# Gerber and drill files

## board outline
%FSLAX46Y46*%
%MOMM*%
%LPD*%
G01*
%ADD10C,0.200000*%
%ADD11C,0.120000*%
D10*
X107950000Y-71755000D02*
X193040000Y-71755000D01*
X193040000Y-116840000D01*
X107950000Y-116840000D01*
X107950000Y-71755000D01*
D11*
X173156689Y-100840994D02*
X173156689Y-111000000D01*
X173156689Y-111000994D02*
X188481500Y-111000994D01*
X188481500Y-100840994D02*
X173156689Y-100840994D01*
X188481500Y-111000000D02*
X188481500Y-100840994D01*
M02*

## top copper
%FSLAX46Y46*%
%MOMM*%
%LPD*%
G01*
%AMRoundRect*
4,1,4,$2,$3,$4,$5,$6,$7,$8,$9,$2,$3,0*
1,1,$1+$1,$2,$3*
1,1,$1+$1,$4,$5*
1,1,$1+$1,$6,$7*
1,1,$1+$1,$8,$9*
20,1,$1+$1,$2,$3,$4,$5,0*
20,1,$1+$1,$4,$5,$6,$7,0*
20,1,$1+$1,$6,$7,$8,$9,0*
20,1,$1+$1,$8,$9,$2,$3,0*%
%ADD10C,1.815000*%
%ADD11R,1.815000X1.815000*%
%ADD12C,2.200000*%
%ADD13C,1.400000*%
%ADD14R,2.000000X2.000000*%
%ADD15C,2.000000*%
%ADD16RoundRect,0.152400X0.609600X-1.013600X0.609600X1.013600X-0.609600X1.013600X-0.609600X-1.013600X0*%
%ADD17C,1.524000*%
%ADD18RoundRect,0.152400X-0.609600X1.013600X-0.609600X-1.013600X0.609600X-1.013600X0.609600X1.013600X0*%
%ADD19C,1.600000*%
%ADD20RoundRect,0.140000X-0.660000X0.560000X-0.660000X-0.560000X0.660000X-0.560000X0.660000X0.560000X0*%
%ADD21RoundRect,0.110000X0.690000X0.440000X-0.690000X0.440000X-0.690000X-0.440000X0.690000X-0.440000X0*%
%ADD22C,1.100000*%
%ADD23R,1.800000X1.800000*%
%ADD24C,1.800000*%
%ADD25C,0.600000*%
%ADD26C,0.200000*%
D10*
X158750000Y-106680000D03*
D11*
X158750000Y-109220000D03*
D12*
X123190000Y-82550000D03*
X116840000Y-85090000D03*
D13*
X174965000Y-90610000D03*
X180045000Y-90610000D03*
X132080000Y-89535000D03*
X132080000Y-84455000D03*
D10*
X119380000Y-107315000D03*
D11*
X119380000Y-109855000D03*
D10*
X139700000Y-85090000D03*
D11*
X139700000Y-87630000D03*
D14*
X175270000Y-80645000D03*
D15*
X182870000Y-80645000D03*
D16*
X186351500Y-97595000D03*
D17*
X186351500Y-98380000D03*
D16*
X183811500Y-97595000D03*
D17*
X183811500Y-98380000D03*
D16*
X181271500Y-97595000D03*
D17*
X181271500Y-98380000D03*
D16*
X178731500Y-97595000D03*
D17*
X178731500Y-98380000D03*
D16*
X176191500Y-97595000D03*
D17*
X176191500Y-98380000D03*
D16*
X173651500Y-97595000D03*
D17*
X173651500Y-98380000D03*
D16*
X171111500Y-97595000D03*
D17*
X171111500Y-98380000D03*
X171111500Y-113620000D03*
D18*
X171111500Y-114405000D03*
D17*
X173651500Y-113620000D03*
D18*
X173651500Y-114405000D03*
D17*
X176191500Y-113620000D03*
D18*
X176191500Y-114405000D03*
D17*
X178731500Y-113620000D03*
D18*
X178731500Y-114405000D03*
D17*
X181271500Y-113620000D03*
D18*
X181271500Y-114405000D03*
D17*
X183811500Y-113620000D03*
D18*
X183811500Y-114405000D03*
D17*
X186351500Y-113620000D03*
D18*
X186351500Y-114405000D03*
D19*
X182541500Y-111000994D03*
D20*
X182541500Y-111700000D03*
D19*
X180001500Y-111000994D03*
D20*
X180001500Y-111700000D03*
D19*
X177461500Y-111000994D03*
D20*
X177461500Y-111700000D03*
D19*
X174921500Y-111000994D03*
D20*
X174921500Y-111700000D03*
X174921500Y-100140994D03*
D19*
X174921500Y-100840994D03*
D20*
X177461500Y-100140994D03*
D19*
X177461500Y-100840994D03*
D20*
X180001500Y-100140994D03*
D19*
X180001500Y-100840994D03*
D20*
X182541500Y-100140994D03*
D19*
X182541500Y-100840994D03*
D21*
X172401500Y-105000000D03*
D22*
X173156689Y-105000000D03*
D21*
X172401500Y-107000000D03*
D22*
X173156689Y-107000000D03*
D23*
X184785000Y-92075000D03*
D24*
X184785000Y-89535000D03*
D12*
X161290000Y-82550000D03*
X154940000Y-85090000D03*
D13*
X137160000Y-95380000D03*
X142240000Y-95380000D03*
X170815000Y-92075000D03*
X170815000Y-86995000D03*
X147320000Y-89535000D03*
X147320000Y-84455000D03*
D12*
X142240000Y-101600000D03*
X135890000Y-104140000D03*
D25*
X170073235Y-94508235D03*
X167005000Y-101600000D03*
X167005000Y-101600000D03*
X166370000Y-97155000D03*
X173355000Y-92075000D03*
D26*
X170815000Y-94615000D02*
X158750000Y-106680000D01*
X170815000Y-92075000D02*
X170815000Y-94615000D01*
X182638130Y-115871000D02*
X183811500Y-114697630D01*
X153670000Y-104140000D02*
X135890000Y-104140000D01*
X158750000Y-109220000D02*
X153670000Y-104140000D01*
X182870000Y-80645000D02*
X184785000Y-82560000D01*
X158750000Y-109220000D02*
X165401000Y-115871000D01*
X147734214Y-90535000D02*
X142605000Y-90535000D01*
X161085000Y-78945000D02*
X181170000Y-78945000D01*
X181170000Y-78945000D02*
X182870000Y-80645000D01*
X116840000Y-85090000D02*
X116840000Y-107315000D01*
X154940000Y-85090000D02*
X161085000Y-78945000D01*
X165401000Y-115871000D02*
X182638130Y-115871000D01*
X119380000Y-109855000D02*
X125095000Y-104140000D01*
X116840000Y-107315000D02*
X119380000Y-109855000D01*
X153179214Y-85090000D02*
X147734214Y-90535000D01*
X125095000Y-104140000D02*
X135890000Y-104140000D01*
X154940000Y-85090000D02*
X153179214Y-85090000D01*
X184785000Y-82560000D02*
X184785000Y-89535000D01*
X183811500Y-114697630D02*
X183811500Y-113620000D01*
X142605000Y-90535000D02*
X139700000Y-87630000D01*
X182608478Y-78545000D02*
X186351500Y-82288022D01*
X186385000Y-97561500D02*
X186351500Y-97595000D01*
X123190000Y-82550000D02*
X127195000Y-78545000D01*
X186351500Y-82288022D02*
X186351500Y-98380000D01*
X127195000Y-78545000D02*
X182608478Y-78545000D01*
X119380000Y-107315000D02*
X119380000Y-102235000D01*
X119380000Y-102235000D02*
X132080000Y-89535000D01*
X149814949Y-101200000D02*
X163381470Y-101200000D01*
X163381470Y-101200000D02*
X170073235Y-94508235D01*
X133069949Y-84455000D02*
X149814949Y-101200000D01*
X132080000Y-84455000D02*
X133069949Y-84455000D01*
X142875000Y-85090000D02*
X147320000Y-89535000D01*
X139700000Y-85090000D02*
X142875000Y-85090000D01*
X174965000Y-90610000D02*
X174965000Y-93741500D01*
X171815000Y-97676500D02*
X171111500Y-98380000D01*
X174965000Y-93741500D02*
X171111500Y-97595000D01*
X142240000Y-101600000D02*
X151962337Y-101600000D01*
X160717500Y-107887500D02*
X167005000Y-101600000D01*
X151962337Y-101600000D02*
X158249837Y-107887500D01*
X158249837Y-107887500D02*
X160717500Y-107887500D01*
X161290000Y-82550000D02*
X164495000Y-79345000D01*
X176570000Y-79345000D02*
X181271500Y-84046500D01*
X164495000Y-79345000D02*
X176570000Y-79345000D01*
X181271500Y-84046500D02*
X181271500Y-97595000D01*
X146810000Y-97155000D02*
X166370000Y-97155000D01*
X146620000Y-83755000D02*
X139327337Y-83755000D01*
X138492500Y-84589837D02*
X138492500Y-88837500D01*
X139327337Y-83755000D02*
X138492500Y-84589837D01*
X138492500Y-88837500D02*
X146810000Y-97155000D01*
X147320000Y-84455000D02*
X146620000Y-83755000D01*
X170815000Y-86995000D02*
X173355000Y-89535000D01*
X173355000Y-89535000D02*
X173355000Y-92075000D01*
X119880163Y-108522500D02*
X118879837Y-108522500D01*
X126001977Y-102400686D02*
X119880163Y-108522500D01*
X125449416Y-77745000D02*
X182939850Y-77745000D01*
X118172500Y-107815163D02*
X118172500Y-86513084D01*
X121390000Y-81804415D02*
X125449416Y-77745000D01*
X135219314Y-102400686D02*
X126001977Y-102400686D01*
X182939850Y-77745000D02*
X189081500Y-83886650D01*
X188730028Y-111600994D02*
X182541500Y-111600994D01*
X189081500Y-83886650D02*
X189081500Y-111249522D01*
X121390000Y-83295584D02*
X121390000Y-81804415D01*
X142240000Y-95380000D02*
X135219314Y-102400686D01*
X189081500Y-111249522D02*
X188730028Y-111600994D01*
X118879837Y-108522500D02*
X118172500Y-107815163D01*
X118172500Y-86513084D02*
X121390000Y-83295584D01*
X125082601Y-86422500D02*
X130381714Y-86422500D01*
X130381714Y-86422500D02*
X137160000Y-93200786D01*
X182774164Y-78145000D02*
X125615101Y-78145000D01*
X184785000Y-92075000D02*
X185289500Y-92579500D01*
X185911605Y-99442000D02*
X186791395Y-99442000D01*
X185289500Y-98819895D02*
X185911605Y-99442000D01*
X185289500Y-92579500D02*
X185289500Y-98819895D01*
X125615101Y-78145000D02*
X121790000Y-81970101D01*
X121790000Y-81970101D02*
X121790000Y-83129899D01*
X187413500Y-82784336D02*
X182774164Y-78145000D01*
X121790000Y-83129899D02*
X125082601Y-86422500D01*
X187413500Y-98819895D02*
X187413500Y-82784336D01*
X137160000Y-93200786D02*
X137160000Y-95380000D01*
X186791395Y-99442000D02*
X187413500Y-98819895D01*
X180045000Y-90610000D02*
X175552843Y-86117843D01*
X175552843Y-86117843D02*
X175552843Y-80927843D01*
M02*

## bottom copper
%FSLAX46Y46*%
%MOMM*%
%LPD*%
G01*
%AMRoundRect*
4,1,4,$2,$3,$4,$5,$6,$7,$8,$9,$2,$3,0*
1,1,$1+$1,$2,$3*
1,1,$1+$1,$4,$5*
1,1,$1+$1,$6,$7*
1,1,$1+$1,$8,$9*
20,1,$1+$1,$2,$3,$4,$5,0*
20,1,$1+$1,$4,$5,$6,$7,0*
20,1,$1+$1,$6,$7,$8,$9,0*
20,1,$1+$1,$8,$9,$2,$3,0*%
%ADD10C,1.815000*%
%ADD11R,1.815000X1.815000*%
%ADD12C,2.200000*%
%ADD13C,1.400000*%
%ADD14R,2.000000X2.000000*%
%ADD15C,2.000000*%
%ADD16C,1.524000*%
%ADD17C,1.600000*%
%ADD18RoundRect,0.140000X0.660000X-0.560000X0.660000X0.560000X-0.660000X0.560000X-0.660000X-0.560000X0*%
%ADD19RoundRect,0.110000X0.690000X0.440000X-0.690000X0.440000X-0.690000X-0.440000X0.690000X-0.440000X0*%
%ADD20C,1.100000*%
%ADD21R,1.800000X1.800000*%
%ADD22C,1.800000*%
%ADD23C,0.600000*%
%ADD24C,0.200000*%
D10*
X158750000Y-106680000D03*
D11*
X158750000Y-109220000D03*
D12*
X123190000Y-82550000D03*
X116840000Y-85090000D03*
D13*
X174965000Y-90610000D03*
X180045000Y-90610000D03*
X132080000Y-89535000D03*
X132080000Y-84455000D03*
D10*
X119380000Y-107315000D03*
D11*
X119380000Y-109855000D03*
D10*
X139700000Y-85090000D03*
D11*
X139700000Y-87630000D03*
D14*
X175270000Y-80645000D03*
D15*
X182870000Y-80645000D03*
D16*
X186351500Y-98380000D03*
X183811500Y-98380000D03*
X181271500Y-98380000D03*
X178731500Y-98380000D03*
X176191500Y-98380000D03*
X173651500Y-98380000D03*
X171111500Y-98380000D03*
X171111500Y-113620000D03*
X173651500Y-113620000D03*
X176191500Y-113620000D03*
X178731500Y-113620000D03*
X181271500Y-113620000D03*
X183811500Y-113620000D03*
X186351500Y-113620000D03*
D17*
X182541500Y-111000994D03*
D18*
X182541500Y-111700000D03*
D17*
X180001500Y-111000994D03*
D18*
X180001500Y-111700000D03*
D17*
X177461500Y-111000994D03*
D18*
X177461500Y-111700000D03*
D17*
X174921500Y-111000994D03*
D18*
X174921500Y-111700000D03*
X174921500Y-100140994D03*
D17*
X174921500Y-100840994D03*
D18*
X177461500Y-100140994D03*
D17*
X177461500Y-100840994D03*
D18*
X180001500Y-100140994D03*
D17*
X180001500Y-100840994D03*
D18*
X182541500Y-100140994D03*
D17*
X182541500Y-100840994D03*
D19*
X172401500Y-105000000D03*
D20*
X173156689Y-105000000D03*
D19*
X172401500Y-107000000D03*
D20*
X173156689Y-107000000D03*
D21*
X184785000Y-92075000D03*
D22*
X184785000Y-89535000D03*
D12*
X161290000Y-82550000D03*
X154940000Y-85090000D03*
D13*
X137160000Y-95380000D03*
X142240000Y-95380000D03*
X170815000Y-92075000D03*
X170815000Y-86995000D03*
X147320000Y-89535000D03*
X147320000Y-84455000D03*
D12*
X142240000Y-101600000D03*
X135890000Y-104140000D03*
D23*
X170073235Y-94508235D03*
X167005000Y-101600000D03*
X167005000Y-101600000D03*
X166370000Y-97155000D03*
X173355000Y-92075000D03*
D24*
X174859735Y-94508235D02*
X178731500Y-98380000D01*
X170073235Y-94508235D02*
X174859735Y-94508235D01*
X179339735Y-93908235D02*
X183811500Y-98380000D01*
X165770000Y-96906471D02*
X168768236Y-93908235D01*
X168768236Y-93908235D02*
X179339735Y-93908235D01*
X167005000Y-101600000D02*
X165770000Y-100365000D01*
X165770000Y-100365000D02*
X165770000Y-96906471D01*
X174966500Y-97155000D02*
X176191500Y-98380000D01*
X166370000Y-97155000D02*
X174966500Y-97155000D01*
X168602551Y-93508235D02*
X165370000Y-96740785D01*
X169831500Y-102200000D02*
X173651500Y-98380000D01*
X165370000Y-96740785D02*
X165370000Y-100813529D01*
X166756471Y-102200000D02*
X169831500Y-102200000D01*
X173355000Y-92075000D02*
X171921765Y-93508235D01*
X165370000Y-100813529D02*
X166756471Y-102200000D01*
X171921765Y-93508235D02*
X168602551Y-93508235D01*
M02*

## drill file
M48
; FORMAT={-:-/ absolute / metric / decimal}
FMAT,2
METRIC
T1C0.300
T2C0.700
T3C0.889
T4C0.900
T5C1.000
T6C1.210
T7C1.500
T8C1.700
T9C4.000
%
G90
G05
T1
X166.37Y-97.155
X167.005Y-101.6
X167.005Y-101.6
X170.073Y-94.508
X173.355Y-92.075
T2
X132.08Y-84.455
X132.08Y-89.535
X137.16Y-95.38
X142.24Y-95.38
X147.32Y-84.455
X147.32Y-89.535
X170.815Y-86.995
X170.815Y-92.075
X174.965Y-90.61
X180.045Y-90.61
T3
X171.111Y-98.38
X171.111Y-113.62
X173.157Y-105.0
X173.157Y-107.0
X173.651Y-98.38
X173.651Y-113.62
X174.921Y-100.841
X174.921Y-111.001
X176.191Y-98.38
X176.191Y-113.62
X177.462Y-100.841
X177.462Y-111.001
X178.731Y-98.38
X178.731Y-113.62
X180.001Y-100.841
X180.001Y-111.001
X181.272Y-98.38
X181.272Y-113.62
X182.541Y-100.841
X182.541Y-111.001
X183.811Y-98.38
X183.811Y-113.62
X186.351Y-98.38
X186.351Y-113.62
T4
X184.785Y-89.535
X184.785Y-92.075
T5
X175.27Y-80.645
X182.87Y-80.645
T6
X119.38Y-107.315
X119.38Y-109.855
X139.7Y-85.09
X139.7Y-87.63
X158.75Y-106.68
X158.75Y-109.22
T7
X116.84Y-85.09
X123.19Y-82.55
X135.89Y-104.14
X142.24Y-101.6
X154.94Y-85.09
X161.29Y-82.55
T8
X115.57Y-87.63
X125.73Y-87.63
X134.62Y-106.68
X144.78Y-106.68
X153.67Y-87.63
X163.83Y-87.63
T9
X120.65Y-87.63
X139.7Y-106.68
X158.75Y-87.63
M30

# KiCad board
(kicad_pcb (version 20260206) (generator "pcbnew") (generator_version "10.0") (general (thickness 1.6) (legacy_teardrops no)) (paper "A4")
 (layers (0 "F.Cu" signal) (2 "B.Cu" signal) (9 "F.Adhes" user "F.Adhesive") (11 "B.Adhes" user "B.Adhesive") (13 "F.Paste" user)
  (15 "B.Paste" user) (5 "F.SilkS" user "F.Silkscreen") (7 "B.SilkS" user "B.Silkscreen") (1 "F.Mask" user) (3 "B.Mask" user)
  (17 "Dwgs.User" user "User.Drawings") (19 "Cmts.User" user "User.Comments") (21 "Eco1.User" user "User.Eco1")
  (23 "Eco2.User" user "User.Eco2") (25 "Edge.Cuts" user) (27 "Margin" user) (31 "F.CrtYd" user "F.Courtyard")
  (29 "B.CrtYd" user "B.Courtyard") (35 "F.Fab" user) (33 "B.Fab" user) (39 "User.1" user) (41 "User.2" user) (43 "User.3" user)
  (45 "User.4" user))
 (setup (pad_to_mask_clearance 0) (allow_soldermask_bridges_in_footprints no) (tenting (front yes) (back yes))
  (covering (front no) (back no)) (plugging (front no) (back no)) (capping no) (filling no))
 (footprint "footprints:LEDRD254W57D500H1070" (layer "F.Cu") (at 158.75 107.95 90)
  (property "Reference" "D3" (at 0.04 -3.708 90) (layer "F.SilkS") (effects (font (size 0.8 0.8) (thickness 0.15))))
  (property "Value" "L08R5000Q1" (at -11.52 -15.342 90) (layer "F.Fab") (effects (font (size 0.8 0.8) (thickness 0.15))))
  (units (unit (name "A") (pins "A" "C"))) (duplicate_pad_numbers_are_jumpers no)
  (pad "A" thru_hole circle (at 1.27 0 90) (size 1.815 1.815) (drill 1.21) (layers "*.Cu" "*.Mask") (remove_unused_layers no)
   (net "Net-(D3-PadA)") (solder_mask_margin 0.102))
  (pad "C" thru_hole rect (at -1.27 0 90) (size 1.815 1.815) (drill 1.21) (layers "*.Cu" "*.Mask") (remove_unused_layers no) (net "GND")
   (solder_mask_margin 0.102)))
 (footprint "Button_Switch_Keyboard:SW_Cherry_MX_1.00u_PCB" (layer "F.Cu") (at 123.19 82.55)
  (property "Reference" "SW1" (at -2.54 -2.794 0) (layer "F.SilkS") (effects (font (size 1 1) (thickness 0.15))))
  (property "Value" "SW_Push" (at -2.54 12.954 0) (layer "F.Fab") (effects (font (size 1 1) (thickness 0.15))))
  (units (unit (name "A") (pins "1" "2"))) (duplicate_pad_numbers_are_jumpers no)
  (pad "" np_thru_hole circle (at -7.62 5.08) (size 1.7 1.7) (drill 1.7) (layers "*.Cu" "*.Mask"))
  (pad "" np_thru_hole circle (at -2.54 5.08) (size 4 4) (drill 4) (layers "*.Cu" "*.Mask"))
  (pad "" np_thru_hole circle (at 2.54 5.08) (size 1.7 1.7) (drill 1.7) (layers "*.Cu" "*.Mask"))
  (pad "1" thru_hole circle (at 0 0) (size 2.2 2.2) (drill 1.5) (layers "*.Cu" "*.Mask") (remove_unused_layers no) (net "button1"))
  (pad "2" thru_hole circle (at -6.35 2.54) (size 2.2 2.2) (drill 1.5) (layers "*.Cu" "*.Mask") (remove_unused_layers no) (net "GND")))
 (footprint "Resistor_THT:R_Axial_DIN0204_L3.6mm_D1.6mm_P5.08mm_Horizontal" (layer "F.Cu") (at 174.965 90.61)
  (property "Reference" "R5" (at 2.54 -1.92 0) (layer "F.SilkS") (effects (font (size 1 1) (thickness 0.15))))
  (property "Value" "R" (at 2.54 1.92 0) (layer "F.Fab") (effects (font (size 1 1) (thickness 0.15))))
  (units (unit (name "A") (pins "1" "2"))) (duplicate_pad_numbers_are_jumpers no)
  (pad "1" thru_hole circle (at 0 0) (size 1.4 1.4) (drill 0.7) (layers "*.Cu" "*.Mask") (remove_unused_layers no) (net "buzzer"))
  (pad "2" thru_hole circle (at 5.08 0) (size 1.4 1.4) (drill 0.7) (layers "*.Cu" "*.Mask") (remove_unused_layers no) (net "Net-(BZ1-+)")))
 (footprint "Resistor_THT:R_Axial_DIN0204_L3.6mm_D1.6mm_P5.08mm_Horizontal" (layer "F.Cu") (at 132.08 89.535 90)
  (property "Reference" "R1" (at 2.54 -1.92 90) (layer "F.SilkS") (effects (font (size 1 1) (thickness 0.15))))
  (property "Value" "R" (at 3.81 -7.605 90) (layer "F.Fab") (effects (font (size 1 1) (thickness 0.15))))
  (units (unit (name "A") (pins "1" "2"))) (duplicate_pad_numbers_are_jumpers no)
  (pad "1" thru_hole circle (at 0 0 90) (size 1.4 1.4) (drill 0.7) (layers "*.Cu" "*.Mask") (remove_unused_layers no) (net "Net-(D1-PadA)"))
  (pad "2" thru_hole circle (at 5.08 0 90) (size 1.4 1.4) (drill 0.7) (layers "*.Cu" "*.Mask") (remove_unused_layers no) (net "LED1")))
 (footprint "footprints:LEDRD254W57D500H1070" (layer "F.Cu") (at 119.38 108.585 90)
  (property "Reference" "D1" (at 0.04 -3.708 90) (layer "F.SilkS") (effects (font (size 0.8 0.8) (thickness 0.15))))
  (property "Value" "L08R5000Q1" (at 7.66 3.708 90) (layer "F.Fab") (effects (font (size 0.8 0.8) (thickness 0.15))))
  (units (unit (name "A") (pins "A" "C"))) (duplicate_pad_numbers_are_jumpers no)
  (pad "A" thru_hole circle (at 1.27 0 90) (size 1.815 1.815) (drill 1.21) (layers "*.Cu" "*.Mask") (remove_unused_layers no)
   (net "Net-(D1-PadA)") (solder_mask_margin 0.102))
  (pad "C" thru_hole rect (at -1.27 0 90) (size 1.815 1.815) (drill 1.21) (layers "*.Cu" "*.Mask") (remove_unused_layers no) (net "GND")
   (solder_mask_margin 0.102)))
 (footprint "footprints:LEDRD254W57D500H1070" (layer "F.Cu") (at 139.7 86.36 90)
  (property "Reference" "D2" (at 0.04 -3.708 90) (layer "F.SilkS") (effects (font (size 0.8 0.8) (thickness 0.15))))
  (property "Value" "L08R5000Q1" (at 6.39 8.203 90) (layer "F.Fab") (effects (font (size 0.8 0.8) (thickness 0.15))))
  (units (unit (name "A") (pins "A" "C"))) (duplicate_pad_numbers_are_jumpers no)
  (pad "A" thru_hole circle (at 1.27 0 90) (size 1.815 1.815) (drill 1.21) (layers "*.Cu" "*.Mask") (remove_unused_layers no)
   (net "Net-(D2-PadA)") (solder_mask_margin 0.102))
  (pad "C" thru_hole rect (at -1.27 0 90) (size 1.815 1.815) (drill 1.21) (layers "*.Cu" "*.Mask") (remove_unused_layers no) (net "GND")
   (solder_mask_margin 0.102)))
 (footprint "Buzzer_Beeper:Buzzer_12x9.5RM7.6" (layer "F.Cu") (at 175.27 80.645)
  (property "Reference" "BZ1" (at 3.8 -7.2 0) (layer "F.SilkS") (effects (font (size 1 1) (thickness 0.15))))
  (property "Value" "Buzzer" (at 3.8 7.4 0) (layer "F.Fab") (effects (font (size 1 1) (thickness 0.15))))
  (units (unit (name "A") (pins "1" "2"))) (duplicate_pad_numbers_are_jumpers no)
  (pad "1" thru_hole rect (at 0 0) (size 2 2) (drill 1) (layers "*.Cu" "*.Mask") (remove_unused_layers no) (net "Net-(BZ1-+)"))
  (pad "2" thru_hole circle (at 7.6 0) (size 2 2) (drill 1) (layers "*.Cu" "*.Mask") (remove_unused_layers no) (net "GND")))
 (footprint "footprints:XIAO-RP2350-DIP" (layer "F.Cu") (at 178.7315 106)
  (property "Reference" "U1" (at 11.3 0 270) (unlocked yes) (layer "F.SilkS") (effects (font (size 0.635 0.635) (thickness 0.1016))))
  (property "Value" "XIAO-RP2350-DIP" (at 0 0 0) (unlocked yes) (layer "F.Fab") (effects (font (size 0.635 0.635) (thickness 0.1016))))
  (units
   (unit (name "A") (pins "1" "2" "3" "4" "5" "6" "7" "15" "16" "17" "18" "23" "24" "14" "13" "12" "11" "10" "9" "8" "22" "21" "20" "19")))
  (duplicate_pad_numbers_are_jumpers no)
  (fp_line (start -5.574811 -5.159006) (end -5.574811 5) (stroke (width 0.12) (type default)) (layer "Edge.Cuts"))
  (fp_line (start -5.574811 5.000994) (end 9.75 5.000994) (stroke (width 0.12) (type default)) (layer "Edge.Cuts"))
  (fp_line (start 9.75 -5.159006) (end -5.574811 -5.159006) (stroke (width 0.12) (type default)) (layer "Edge.Cuts"))
  (fp_line (start 9.75 5) (end 9.75 -5.159006) (stroke (width 0.12) (type default)) (layer "Edge.Cuts"))
  (pad "1" smd roundrect (at 7.62 -8.405 90) (size 2.332 1.524) (layers "F.Cu" "F.Mask") (roundrect_rratio 0.1) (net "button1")
   (thermal_bridge_angle 45))
  (pad "1" thru_hole circle (at 7.62 -7.62 90) (size 1.524 1.524) (drill 0.889) (layers "*.Cu" "*.Mask") (remove_unused_layers no)
   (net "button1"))
  (pad "2" smd roundrect (at 5.08 -8.405 90) (size 2.332 1.524) (layers "F.Cu" "F.Mask") (roundrect_rratio 0.1) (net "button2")
   (thermal_bridge_angle 45))
  (pad "2" thru_hole circle (at 5.08 -7.62 90) (size 1.524 1.524) (drill 0.889) (layers "*.Cu" "*.Mask") (remove_unused_layers no)
   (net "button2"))
  (pad "3" smd roundrect (at 2.54 -8.405 90) (size 2.332 1.524) (layers "F.Cu" "F.Mask") (roundrect_rratio 0.1) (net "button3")
   (thermal_bridge_angle 45))
  (pad "3" thru_hole circle (at 2.54 -7.62 90) (size 1.524 1.524) (drill 0.889) (layers "*.Cu" "*.Mask") (remove_unused_layers no)
   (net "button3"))
  (pad "4" smd roundrect (at 0 -8.405 90) (size 2.332 1.524) (layers "F.Cu" "F.Mask") (roundrect_rratio 0.1) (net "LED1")
   (thermal_bridge_angle 45))
  (pad "4" thru_hole circle (at 0 -7.62 90) (size 1.524 1.524) (drill 0.889) (layers "*.Cu" "*.Mask") (remove_unused_layers no) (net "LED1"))
  (pad "5" smd roundrect (at -2.54 -8.405 90) (size 2.332 1.524) (layers "F.Cu" "F.Mask") (roundrect_rratio 0.1) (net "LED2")
   (thermal_bridge_angle 45))
  (pad "5" thru_hole circle (at -2.54 -7.62 90) (size 1.524 1.524) (drill 0.889) (layers "*.Cu" "*.Mask") (remove_unused_layers no)
   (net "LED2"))
  (pad "6" smd roundrect (at -5.08 -8.405 90) (size 2.332 1.524) (layers "F.Cu" "F.Mask") (roundrect_rratio 0.1) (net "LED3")
   (thermal_bridge_angle 45))
  (pad "6" thru_hole circle (at -5.08 -7.62 90) (size 1.524 1.524) (drill 0.889) (layers "*.Cu" "*.Mask") (remove_unused_layers no)
   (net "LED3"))
  (pad "7" smd roundrect (at -7.62 -8.405 90) (size 2.332 1.524) (layers "F.Cu" "F.Mask") (roundrect_rratio 0.1) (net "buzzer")
   (thermal_bridge_angle 45))
  (pad "7" thru_hole circle (at -7.62 -7.62 90) (size 1.524 1.524) (drill 0.889) (layers "*.Cu" "*.Mask") (remove_unused_layers no)
   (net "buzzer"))
  (pad "8" thru_hole circle (at -7.62 7.62 270) (size 1.524 1.524) (drill 0.889) (layers "*.Cu" "*.Mask") (remove_unused_layers no)
   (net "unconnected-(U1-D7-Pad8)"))
  (pad "8" smd roundrect (at -7.62 8.405 270) (size 2.332 1.524) (layers "F.Cu" "F.Mask") (roundrect_rratio 0.1)
   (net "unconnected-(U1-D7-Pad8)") (thermal_bridge_angle 45))
  (pad "9" thru_hole circle (at -5.08 7.62 270) (size 1.524 1.524) (drill 0.889) (layers "*.Cu" "*.Mask") (remove_unused_layers no)
   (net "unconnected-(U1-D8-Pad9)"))
  (pad "9" smd roundrect (at -5.08 8.405 270) (size 2.332 1.524) (layers "F.Cu" "F.Mask") (roundrect_rratio 0.1)
   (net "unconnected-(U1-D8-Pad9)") (thermal_bridge_angle 45))
  (pad "10" thru_hole circle (at -2.54 7.62 270) (size 1.524 1.524) (drill 0.889) (layers "*.Cu" "*.Mask") (remove_unused_layers no)
   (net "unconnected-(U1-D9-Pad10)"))
  (pad "10" smd roundrect (at -2.54 8.405 270) (size 2.332 1.524) (layers "F.Cu" "F.Mask") (roundrect_rratio 0.1)
   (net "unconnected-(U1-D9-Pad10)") (thermal_bridge_angle 45))
  (pad "11" thru_hole circle (at 0 7.62 270) (size 1.524 1.524) (drill 0.889) (layers "*.Cu" "*.Mask") (remove_unused_layers no)
   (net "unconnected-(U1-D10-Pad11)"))
  (pad "11" smd roundrect (at 0 8.405 270) (size 2.332 1.524) (layers "F.Cu" "F.Mask") (roundrect_rratio 0.1)
   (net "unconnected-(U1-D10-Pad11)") (thermal_bridge_angle 45))
  (pad "12" thru_hole circle (at 2.54 7.62 270) (size 1.524 1.524) (drill 0.889) (layers "*.Cu" "*.Mask") (remove_unused_layers no)
   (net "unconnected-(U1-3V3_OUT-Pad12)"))
  (pad "12" smd roundrect (at 2.54 8.405 270) (size 2.332 1.524) (layers "F.Cu" "F.Mask") (roundrect_rratio 0.1)
   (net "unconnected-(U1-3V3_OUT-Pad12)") (thermal_bridge_angle 45))
  (pad "13" thru_hole circle (at 5.08 7.62 270) (size 1.524 1.524) (drill 0.889) (layers "*.Cu" "*.Mask") (remove_unused_layers no)
   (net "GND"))
  (pad "13" smd roundrect (at 5.08 8.405 270) (size 2.332 1.524) (layers "F.Cu" "F.Mask") (roundrect_rratio 0.1) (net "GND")
   (thermal_bridge_angle 45))
  (pad "14" thru_hole circle (at 7.62 7.62 270) (size 1.524 1.524) (drill 0.889) (layers "*.Cu" "*.Mask") (remove_unused_layers no)
   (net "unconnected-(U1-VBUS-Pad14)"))
  (pad "14" smd roundrect (at 7.62 8.405 270) (size 2.332 1.524) (layers "F.Cu" "F.Mask") (roundrect_rratio 0.1)
   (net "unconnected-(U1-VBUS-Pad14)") (thermal_bridge_angle 45))
  (pad "15" thru_hole circle (at 3.81 5.000994 90) (size 1.6 1.6) (drill 0.889) (layers "*.Cu" "*.Mask") (remove_unused_layers no)
   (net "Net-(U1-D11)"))
  (pad "15" smd roundrect (at 3.81 5.7 270) (size 1.4 1.6) (layers "F.Cu" "F.Mask") (roundrect_rratio 0.1) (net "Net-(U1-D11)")
   (thermal_bridge_angle 45))
  (pad "15" smd roundrect (at 3.81 5.7 90) (size 1.4 1.6) (layers "B.Cu" "B.Mask" "B.Paste") (roundrect_rratio 0.1) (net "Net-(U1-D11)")
   (thermal_bridge_angle 45))
  (pad "16" thru_hole circle (at 1.27 5.000994 90) (size 1.6 1.6) (drill 0.889) (layers "*.Cu" "*.Mask") (remove_unused_layers no)
   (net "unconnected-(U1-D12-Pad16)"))
  (pad "16" smd roundrect (at 1.27 5.7 270) (size 1.4 1.6) (layers "F.Cu" "F.Mask") (roundrect_rratio 0.1)
   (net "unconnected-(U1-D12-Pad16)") (thermal_bridge_angle 45))
  (pad "16" smd roundrect (at 1.27 5.7 90) (size 1.4 1.6) (layers "B.Cu" "B.Mask" "B.Paste") (roundrect_rratio 0.1)
   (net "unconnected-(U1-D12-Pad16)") (thermal_bridge_angle 45))
  (pad "17" thru_hole circle (at -1.27 5.000994 90) (size 1.6 1.6) (drill 0.889) (layers "*.Cu" "*.Mask") (remove_unused_layers no)
   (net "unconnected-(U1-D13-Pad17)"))
  (pad "17" smd roundrect (at -1.27 5.7 270) (size 1.4 1.6) (layers "F.Cu" "F.Mask") (roundrect_rratio 0.1)
   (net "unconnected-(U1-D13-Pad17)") (thermal_bridge_angle 45))
  (pad "17" smd roundrect (at -1.27 5.7 90) (size 1.4 1.6) (layers "B.Cu" "B.Mask" "B.Paste") (roundrect_rratio 0.1)
   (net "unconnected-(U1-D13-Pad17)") (thermal_bridge_angle 45))
  (pad "18" thru_hole circle (at -3.81 5.000994 90) (size 1.6 1.6) (drill 0.889) (layers "*.Cu" "*.Mask") (remove_unused_layers no)
   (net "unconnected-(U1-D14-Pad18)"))
  (pad "18" smd roundrect (at -3.81 5.7 270) (size 1.4 1.6) (layers "F.Cu" "F.Mask") (roundrect_rratio 0.1)
   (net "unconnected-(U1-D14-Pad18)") (thermal_bridge_angle 45))
  (pad "18" smd roundrect (at -3.81 5.7 90) (size 1.4 1.6) (layers "B.Cu" "B.Mask" "B.Paste") (roundrect_rratio 0.1)
   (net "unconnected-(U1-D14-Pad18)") (thermal_bridge_angle 45))
  (pad "19" smd roundrect (at -3.81 -5.859006 270) (size 1.4 1.6) (layers "F.Cu" "F.Mask") (roundrect_rratio 0.1)
   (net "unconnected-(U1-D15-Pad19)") (thermal_bridge_angle 45))
  (pad "19" smd roundrect (at -3.81 -5.859006 90) (size 1.4 1.6) (layers "B.Cu" "B.Mask" "B.Paste") (roundrect_rratio 0.1)
   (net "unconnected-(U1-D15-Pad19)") (thermal_bridge_angle 45))
  (pad "19" thru_hole circle (at -3.81 -5.159006 90) (size 1.6 1.6) (drill 0.889) (layers "*.Cu" "*.Mask") (remove_unused_layers no)
   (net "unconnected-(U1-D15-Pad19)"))
  (pad "20" smd roundrect (at -1.27 -5.859006 270) (size 1.4 1.6) (layers "F.Cu" "F.Mask") (roundrect_rratio 0.1)
   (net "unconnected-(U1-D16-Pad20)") (thermal_bridge_angle 45))
  (pad "20" smd roundrect (at -1.27 -5.859006 90) (size 1.4 1.6) (layers "B.Cu" "B.Mask" "B.Paste") (roundrect_rratio 0.1)
   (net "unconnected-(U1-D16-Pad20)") (thermal_bridge_angle 45))
  (pad "20" thru_hole circle (at -1.27 -5.159006 90) (size 1.6 1.6) (drill 0.889) (layers "*.Cu" "*.Mask") (remove_unused_layers no)
   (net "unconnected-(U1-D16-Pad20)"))
  (pad "21" smd roundrect (at 1.27 -5.859006 270) (size 1.4 1.6) (layers "F.Cu" "F.Mask") (roundrect_rratio 0.1)
   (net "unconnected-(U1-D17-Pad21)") (thermal_bridge_angle 45))
  (pad "21" smd roundrect (at 1.27 -5.859006 90) (size 1.4 1.6) (layers "B.Cu" "B.Mask" "B.Paste") (roundrect_rratio 0.1)
   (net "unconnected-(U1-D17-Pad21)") (thermal_bridge_angle 45))
  (pad "21" thru_hole circle (at 1.27 -5.159006 90) (size 1.6 1.6) (drill 0.889) (layers "*.Cu" "*.Mask") (remove_unused_layers no)
   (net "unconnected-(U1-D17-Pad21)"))
  (pad "22" smd roundrect (at 3.81 -5.859006 270) (size 1.4 1.6) (layers "F.Cu" "F.Mask") (roundrect_rratio 0.1)
   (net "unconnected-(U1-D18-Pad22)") (thermal_bridge_angle 45))
  (pad "22" smd roundrect (at 3.81 -5.859006 90) (size 1.4 1.6) (layers "B.Cu" "B.Mask" "B.Paste") (roundrect_rratio 0.1)
   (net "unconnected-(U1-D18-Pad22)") (thermal_bridge_angle 45))
  (pad "22" thru_hole circle (at 3.81 -5.159006 90) (size 1.6 1.6) (drill 0.889) (layers "*.Cu" "*.Mask") (remove_unused_layers no)
   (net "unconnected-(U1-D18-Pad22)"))
  (pad "23" smd roundrect (at -6.33 -1 180) (size 1.6 1.1) (layers "F.Cu" "F.Mask") (roundrect_rratio 0.1)
   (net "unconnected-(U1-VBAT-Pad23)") (thermal_bridge_angle 45))
  (pad "23" smd roundrect (at -6.33 -1 180) (size 1.6 1.1) (layers "B.Cu" "B.Mask" "B.Paste") (roundrect_rratio 0.1)
   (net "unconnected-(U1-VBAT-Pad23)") (thermal_bridge_angle 45))
  (pad "23" thru_hole circle (at -5.574811 -1 90) (size 1.1 1.1) (drill 0.889) (layers "*.Cu" "*.Mask") (remove_unused_layers no)
   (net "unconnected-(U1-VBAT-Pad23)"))
  (pad "24" smd roundrect (at -6.33 1 180) (size 1.6 1.1) (layers "F.Cu" "F.Mask") (roundrect_rratio 0.1) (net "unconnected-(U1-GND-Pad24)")
   (thermal_bridge_angle 45))
  (pad "24" smd roundrect (at -6.33 1 180) (size 1.6 1.1) (layers "B.Cu" "B.Mask" "B.Paste") (roundrect_rratio 0.1)
   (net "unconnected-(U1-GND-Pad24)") (thermal_bridge_angle 45))
  (pad "24" thru_hole circle (at -5.574811 1 90) (size 1.1 1.1) (drill 0.889) (layers "*.Cu" "*.Mask") (remove_unused_layers no)
   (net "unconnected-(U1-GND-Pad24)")))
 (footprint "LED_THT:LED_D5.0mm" (layer "F.Cu") (at 184.785 92.075 90)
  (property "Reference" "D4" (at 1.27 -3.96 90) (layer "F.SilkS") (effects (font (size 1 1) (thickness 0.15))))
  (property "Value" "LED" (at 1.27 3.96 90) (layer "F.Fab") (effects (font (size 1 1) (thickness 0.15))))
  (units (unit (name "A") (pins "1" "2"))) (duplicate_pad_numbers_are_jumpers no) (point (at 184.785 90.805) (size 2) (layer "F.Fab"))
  (pad "1" thru_hole rect (at 0 0 90) (size 1.8 1.8) (drill 0.9) (layers "*.Cu" "*.Mask") (remove_unused_layers no) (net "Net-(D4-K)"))
  (pad "2" thru_hole circle (at 2.54 0 90) (size 1.8 1.8) (drill 0.9) (layers "*.Cu" "*.Mask") (remove_unused_layers no) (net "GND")))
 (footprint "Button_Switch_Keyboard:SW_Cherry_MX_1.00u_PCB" (layer "F.Cu") (at 161.29 82.55)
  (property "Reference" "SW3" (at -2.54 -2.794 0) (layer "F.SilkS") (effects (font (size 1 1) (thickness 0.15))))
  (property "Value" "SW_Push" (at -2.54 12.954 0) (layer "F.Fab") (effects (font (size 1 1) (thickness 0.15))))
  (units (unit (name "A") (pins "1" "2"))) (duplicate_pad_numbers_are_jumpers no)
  (pad "" np_thru_hole circle (at -7.62 5.08) (size 1.7 1.7) (drill 1.7) (layers "*.Cu" "*.Mask"))
  (pad "" np_thru_hole circle (at -2.54 5.08) (size 4 4) (drill 4) (layers "*.Cu" "*.Mask"))
  (pad "" np_thru_hole circle (at 2.54 5.08) (size 1.7 1.7) (drill 1.7) (layers "*.Cu" "*.Mask"))
  (pad "1" thru_hole circle (at 0 0) (size 2.2 2.2) (drill 1.5) (layers "*.Cu" "*.Mask") (remove_unused_layers no) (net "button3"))
  (pad "2" thru_hole circle (at -6.35 2.54) (size 2.2 2.2) (drill 1.5) (layers "*.Cu" "*.Mask") (remove_unused_layers no) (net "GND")))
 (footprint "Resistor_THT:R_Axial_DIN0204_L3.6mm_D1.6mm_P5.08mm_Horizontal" (layer "F.Cu") (at 137.16 95.38)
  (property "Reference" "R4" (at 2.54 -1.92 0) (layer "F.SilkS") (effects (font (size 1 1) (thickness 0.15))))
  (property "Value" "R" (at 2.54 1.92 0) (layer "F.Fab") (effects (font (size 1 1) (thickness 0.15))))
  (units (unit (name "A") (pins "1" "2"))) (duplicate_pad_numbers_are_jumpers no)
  (pad "1" thru_hole circle (at 0 0) (size 1.4 1.4) (drill 0.7) (layers "*.Cu" "*.Mask") (remove_unused_layers no) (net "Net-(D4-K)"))
  (pad "2" thru_hole circle (at 5.08 0) (size 1.4 1.4) (drill 0.7) (layers "*.Cu" "*.Mask") (remove_unused_layers no) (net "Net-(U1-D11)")))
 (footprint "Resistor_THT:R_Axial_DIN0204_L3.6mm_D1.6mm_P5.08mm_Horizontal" (layer "F.Cu") (at 170.815 92.075 90)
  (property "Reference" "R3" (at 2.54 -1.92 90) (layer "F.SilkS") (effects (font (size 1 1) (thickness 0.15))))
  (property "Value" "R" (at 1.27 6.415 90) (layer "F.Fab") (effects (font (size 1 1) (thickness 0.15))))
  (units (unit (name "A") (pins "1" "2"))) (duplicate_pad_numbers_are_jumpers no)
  (pad "1" thru_hole circle (at 0 0 90) (size 1.4 1.4) (drill 0.7) (layers "*.Cu" "*.Mask") (remove_unused_layers no) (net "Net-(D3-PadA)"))
  (pad "2" thru_hole circle (at 5.08 0 90) (size 1.4 1.4) (drill 0.7) (layers "*.Cu" "*.Mask") (remove_unused_layers no) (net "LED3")))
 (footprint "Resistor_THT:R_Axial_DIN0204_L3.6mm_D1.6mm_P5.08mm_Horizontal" (layer "F.Cu") (at 147.32 89.535 90)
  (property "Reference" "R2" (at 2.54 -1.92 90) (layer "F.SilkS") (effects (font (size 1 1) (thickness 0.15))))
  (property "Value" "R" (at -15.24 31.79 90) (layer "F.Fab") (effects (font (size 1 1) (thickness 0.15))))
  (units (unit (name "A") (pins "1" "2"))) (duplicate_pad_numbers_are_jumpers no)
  (pad "1" thru_hole circle (at 0 0 90) (size 1.4 1.4) (drill 0.7) (layers "*.Cu" "*.Mask") (remove_unused_layers no) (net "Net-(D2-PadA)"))
  (pad "2" thru_hole circle (at 5.08 0 90) (size 1.4 1.4) (drill 0.7) (layers "*.Cu" "*.Mask") (remove_unused_layers no) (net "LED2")))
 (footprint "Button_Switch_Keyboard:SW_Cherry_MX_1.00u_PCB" (layer "F.Cu") (at 142.24 101.6)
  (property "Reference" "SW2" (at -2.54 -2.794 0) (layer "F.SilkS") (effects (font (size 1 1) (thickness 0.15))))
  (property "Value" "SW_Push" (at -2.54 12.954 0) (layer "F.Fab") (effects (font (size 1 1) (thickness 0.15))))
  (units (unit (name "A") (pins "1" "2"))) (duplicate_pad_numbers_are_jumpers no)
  (pad "" np_thru_hole circle (at -7.62 5.08) (size 1.7 1.7) (drill 1.7) (layers "*.Cu" "*.Mask"))
  (pad "" np_thru_hole circle (at -2.54 5.08) (size 4 4) (drill 4) (layers "*.Cu" "*.Mask"))
  (pad "" np_thru_hole circle (at 2.54 5.08) (size 1.7 1.7) (drill 1.7) (layers "*.Cu" "*.Mask"))
  (pad "1" thru_hole circle (at 0 0) (size 2.2 2.2) (drill 1.5) (layers "*.Cu" "*.Mask") (remove_unused_layers no) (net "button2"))
  (pad "2" thru_hole circle (at -6.35 2.54) (size 2.2 2.2) (drill 1.5) (layers "*.Cu" "*.Mask") (remove_unused_layers no) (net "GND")))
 (gr_rect (start 107.95 71.755) (end 193.04 116.84) (stroke (width 0.2) (type solid)) (fill no) (layer "Edge.Cuts"))
 (segment (start 170.815 94.615) (end 158.75 106.68) (width 0.2) (layer "F.Cu") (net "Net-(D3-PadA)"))
 (segment (start 170.815 92.075) (end 170.815 94.615) (width 0.2) (layer "F.Cu") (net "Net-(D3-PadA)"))
 (segment (start 182.63813 115.871) (end 183.8115 114.69763) (width 0.2) (layer "F.Cu") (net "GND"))
 (segment (start 153.67 104.14) (end 135.89 104.14) (width 0.2) (layer "F.Cu") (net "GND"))
 (segment (start 158.75 109.22) (end 153.67 104.14) (width 0.2) (layer "F.Cu") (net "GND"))
 (segment (start 182.87 80.645) (end 184.785 82.56) (width 0.2) (layer "F.Cu") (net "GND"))
 (segment (start 158.75 109.22) (end 165.401 115.871) (width 0.2) (layer "F.Cu") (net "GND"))
 (segment (start 147.734214 90.535) (end 142.605 90.535) (width 0.2) (layer "F.Cu") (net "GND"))
 (segment (start 161.085 78.945) (end 181.17 78.945) (width 0.2) (layer "F.Cu") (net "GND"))
 (segment (start 181.17 78.945) (end 182.87 80.645) (width 0.2) (layer "F.Cu") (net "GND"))
 (segment (start 116.84 85.09) (end 116.84 107.315) (width 0.2) (layer "F.Cu") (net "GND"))
 (segment (start 154.94 85.09) (end 161.085 78.945) (width 0.2) (layer "F.Cu") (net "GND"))
 (segment (start 165.401 115.871) (end 182.63813 115.871) (width 0.2) (layer "F.Cu") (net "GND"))
 (segment (start 119.38 109.855) (end 125.095 104.14) (width 0.2) (layer "F.Cu") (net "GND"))
 (segment (start 116.84 107.315) (end 119.38 109.855) (width 0.2) (layer "F.Cu") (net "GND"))
 (segment (start 153.179214 85.09) (end 147.734214 90.535) (width 0.2) (layer "F.Cu") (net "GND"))
 (segment (start 125.095 104.14) (end 135.89 104.14) (width 0.2) (layer "F.Cu") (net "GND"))
 (segment (start 154.94 85.09) (end 153.179214 85.09) (width 0.2) (layer "F.Cu") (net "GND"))
 (segment (start 184.785 82.56) (end 184.785 89.535) (width 0.2) (layer "F.Cu") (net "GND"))
 (segment (start 183.8115 114.69763) (end 183.8115 113.62) (width 0.2) (layer "F.Cu") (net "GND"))
 (segment (start 142.605 90.535) (end 139.7 87.63) (width 0.2) (layer "F.Cu") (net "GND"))
 (segment (start 182.608478 78.545) (end 186.3515 82.288022) (width 0.2) (layer "F.Cu") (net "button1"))
 (segment (start 186.385 97.5615) (end 186.3515 97.595) (width 0.2) (layer "F.Cu") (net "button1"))
 (segment (start 123.19 82.55) (end 127.195 78.545) (width 0.2) (layer "F.Cu") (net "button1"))
 (segment (start 186.3515 82.288022) (end 186.3515 98.38) (width 0.2) (layer "F.Cu") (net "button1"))
 (segment (start 127.195 78.545) (end 182.608478 78.545) (width 0.2) (layer "F.Cu") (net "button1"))
 (segment (start 119.38 107.315) (end 119.38 102.235) (width 0.2) (layer "F.Cu") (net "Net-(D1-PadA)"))
 (segment (start 119.38 102.235) (end 132.08 89.535) (width 0.2) (layer "F.Cu") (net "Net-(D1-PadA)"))
 (segment (start 149.814949 101.2) (end 163.38147 101.2) (width 0.2) (layer "F.Cu") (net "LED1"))
 (segment (start 163.38147 101.2) (end 170.073235 94.508235) (width 0.2) (layer "F.Cu") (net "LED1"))
 (segment (start 133.069949 84.455) (end 149.814949 101.2) (width 0.2) (layer "F.Cu") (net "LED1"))
 (segment (start 132.08 84.455) (end 133.069949 84.455) (width 0.2) (layer "F.Cu") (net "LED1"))
 (via (at 170.073235 94.508235) (size 0.6) (drill 0.3) (layers "F.Cu" "B.Cu") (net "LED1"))
 (segment (start 174.859735 94.508235) (end 178.7315 98.38) (width 0.2) (layer "B.Cu") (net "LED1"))
 (segment (start 170.073235 94.508235) (end 174.859735 94.508235) (width 0.2) (layer "B.Cu") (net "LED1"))
 (segment (start 142.875 85.09) (end 147.32 89.535) (width 0.2) (layer "F.Cu") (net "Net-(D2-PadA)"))
 (segment (start 139.7 85.09) (end 142.875 85.09) (width 0.2) (layer "F.Cu") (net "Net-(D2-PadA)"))
 (segment (start 174.965 90.61) (end 174.965 93.7415) (width 0.2) (layer "F.Cu") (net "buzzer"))
 (segment (start 171.815 97.6765) (end 171.1115 98.38) (width 0.2) (layer "F.Cu") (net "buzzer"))
 (segment (start 174.965 93.7415) (end 171.1115 97.595) (width 0.2) (layer "F.Cu") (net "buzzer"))
 (segment (start 142.24 101.6) (end 151.962337 101.6) (width 0.2) (layer "F.Cu") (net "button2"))
 (segment (start 160.7175 107.8875) (end 167.005 101.6) (width 0.2) (layer "F.Cu") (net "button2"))
 (segment (start 151.962337 101.6) (end 158.249837 107.8875) (width 0.2) (layer "F.Cu") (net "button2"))
 (segment (start 158.249837 107.8875) (end 160.7175 107.8875) (width 0.2) (layer "F.Cu") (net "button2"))
 (via (at 167.005 101.6) (size 0.6) (drill 0.3) (layers "F.Cu" "B.Cu") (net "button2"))
 (via (at 167.005 101.6) (size 0.6) (drill 0.3) (layers "F.Cu" "B.Cu") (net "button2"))
 (segment (start 179.339735 93.908235) (end 183.8115 98.38) (width 0.2) (layer "B.Cu") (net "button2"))
 (segment (start 165.77 96.906471) (end 168.768236 93.908235) (width 0.2) (layer "B.Cu") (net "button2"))
 (segment (start 168.768236 93.908235) (end 179.339735 93.908235) (width 0.2) (layer "B.Cu") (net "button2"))
 (segment (start 167.005 101.6) (end 165.77 100.365) (width 0.2) (layer "B.Cu") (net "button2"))
 (segment (start 165.77 100.365) (end 165.77 96.906471) (width 0.2) (layer "B.Cu") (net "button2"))
 (segment (start 161.29 82.55) (end 164.495 79.345) (width 0.2) (layer "F.Cu") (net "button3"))
 (segment (start 176.57 79.345) (end 181.2715 84.0465) (width 0.2) (layer "F.Cu") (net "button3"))
 (segment (start 164.495 79.345) (end 176.57 79.345) (width 0.2) (layer "F.Cu") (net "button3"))
 (segment (start 181.2715 84.0465) (end 181.2715 97.595) (width 0.2) (layer "F.Cu") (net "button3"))
 (segment (start 146.81 97.155) (end 166.37 97.155) (width 0.2) (layer "F.Cu") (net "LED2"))
 (segment (start 146.62 83.755) (end 139.327337 83.755) (width 0.2) (layer "F.Cu") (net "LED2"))
 (segment (start 138.4925 84.589837) (end 138.4925 88.8375) (width 0.2) (layer "F.Cu") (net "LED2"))
 (segment (start 139.327337 83.755) (end 138.4925 84.589837) (width 0.2) (layer "F.Cu") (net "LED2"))
 (segment (start 138.4925 88.8375) (end 146.81 97.155) (width 0.2) (layer "F.Cu") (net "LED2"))
 (segment (start 147.32 84.455) (end 146.62 83.755) (width 0.2) (layer "F.Cu") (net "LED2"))
 (via (at 166.37 97.155) (size 0.6) (drill 0.3) (layers "F.Cu" "B.Cu") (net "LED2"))
 (segment (start 174.9665 97.155) (end 176.1915 98.38) (width 0.2) (layer "B.Cu") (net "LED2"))
 (segment (start 166.37 97.155) (end 174.9665 97.155) (width 0.2) (layer "B.Cu") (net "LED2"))
 (segment (start 170.815 86.995) (end 173.355 89.535) (width 0.2) (layer "F.Cu") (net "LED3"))
 (segment (start 173.355 89.535) (end 173.355 92.075) (width 0.2) (layer "F.Cu") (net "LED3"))
 (via (at 173.355 92.075) (size 0.6) (drill 0.3) (layers "F.Cu" "B.Cu") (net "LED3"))
 (segment (start 168.602551 93.508235) (end 165.37 96.740785) (width 0.2) (layer "B.Cu") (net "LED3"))
 (segment (start 169.8315 102.2) (end 173.6515 98.38) (width 0.2) (layer "B.Cu") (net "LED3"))
 (segment (start 165.37 96.740785) (end 165.37 100.813529) (width 0.2) (layer "B.Cu") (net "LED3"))
 (segment (start 166.756471 102.2) (end 169.8315 102.2) (width 0.2) (layer "B.Cu") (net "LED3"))
 (segment (start 173.355 92.075) (end 171.921765 93.508235) (width 0.2) (layer "B.Cu") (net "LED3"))
 (segment (start 165.37 100.813529) (end 166.756471 102.2) (width 0.2) (layer "B.Cu") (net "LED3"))
 (segment (start 171.921765 93.508235) (end 168.602551 93.508235) (width 0.2) (layer "B.Cu") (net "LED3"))
 (segment (start 119.880163 108.5225) (end 118.879837 108.5225) (width 0.2) (layer "F.Cu") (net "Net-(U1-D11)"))
 (segment (start 126.001977 102.400686) (end 119.880163 108.5225) (width 0.2) (layer "F.Cu") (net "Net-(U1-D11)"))
 (segment (start 125.449416 77.745) (end 182.93985 77.745) (width 0.2) (layer "F.Cu") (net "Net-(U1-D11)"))
 (segment (start 118.1725 107.815163) (end 118.1725 86.513084) (width 0.2) (layer "F.Cu") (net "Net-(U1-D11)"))
 (segment (start 121.39 81.804415) (end 125.449416 77.745) (width 0.2) (layer "F.Cu") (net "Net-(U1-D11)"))
 (segment (start 135.219314 102.400686) (end 126.001977 102.400686) (width 0.2) (layer "F.Cu") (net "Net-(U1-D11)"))
 (segment (start 182.93985 77.745) (end 189.0815 83.88665) (width 0.2) (layer "F.Cu") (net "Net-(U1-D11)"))
 (segment (start 188.730028 111.600994) (end 182.5415 111.600994) (width 0.2) (layer "F.Cu") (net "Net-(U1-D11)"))
 (segment (start 189.0815 83.88665) (end 189.0815 111.249522) (width 0.2) (layer "F.Cu") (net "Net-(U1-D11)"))
 (segment (start 121.39 83.295584) (end 121.39 81.804415) (width 0.2) (layer "F.Cu") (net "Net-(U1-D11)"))
 (segment (start 142.24 95.38) (end 135.219314 102.400686) (width 0.2) (layer "F.Cu") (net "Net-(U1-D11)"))
 (segment (start 189.0815 111.249522) (end 188.730028 111.600994) (width 0.2) (layer "F.Cu") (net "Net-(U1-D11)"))
 (segment (start 118.879837 108.5225) (end 118.1725 107.815163) (width 0.2) (layer "F.Cu") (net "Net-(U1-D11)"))
 (segment (start 118.1725 86.513084) (end 121.39 83.295584) (width 0.2) (layer "F.Cu") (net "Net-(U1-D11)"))
 (segment (start 125.082601 86.4225) (end 130.381714 86.4225) (width 0.2) (layer "F.Cu") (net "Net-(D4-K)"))
 (segment (start 130.381714 86.4225) (end 137.16 93.200786) (width 0.2) (layer "F.Cu") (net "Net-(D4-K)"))
 (segment (start 182.774164 78.145) (end 125.615101 78.145) (width 0.2) (layer "F.Cu") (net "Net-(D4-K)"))
 (segment (start 184.785 92.075) (end 185.2895 92.5795) (width 0.2) (layer "F.Cu") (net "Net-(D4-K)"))
 (segment (start 185.911605 99.442) (end 186.791395 99.442) (width 0.2) (layer "F.Cu") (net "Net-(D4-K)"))
 (segment (start 185.2895 98.819895) (end 185.911605 99.442) (width 0.2) (layer "F.Cu") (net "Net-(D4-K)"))
 (segment (start 185.2895 92.5795) (end 185.2895 98.819895) (width 0.2) (layer "F.Cu") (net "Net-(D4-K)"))
 (segment (start 125.615101 78.145) (end 121.79 81.970101) (width 0.2) (layer "F.Cu") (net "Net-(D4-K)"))
 (segment (start 121.79 81.970101) (end 121.79 83.129899) (width 0.2) (layer "F.Cu") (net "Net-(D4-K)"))
 (segment (start 187.4135 82.784336) (end 182.774164 78.145) (width 0.2) (layer "F.Cu") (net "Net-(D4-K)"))
 (segment (start 121.79 83.129899) (end 125.082601 86.4225) (width 0.2) (layer "F.Cu") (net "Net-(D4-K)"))
 (segment (start 187.4135 98.819895) (end 187.4135 82.784336) (width 0.2) (layer "F.Cu") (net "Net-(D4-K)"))
 (segment (start 137.16 93.200786) (end 137.16 95.38) (width 0.2) (layer "F.Cu") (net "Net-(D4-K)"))
 (segment (start 186.791395 99.442) (end 187.4135 98.819895) (width 0.2) (layer "F.Cu") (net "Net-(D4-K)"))
 (segment (start 180.045 90.61) (end 175.552843 86.117843) (width 0.2) (layer "F.Cu") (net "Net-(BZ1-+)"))
 (segment (start 175.552843 86.117843) (end 175.552843 80.927843) (width 0.2) (layer "F.Cu") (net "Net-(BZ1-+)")))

